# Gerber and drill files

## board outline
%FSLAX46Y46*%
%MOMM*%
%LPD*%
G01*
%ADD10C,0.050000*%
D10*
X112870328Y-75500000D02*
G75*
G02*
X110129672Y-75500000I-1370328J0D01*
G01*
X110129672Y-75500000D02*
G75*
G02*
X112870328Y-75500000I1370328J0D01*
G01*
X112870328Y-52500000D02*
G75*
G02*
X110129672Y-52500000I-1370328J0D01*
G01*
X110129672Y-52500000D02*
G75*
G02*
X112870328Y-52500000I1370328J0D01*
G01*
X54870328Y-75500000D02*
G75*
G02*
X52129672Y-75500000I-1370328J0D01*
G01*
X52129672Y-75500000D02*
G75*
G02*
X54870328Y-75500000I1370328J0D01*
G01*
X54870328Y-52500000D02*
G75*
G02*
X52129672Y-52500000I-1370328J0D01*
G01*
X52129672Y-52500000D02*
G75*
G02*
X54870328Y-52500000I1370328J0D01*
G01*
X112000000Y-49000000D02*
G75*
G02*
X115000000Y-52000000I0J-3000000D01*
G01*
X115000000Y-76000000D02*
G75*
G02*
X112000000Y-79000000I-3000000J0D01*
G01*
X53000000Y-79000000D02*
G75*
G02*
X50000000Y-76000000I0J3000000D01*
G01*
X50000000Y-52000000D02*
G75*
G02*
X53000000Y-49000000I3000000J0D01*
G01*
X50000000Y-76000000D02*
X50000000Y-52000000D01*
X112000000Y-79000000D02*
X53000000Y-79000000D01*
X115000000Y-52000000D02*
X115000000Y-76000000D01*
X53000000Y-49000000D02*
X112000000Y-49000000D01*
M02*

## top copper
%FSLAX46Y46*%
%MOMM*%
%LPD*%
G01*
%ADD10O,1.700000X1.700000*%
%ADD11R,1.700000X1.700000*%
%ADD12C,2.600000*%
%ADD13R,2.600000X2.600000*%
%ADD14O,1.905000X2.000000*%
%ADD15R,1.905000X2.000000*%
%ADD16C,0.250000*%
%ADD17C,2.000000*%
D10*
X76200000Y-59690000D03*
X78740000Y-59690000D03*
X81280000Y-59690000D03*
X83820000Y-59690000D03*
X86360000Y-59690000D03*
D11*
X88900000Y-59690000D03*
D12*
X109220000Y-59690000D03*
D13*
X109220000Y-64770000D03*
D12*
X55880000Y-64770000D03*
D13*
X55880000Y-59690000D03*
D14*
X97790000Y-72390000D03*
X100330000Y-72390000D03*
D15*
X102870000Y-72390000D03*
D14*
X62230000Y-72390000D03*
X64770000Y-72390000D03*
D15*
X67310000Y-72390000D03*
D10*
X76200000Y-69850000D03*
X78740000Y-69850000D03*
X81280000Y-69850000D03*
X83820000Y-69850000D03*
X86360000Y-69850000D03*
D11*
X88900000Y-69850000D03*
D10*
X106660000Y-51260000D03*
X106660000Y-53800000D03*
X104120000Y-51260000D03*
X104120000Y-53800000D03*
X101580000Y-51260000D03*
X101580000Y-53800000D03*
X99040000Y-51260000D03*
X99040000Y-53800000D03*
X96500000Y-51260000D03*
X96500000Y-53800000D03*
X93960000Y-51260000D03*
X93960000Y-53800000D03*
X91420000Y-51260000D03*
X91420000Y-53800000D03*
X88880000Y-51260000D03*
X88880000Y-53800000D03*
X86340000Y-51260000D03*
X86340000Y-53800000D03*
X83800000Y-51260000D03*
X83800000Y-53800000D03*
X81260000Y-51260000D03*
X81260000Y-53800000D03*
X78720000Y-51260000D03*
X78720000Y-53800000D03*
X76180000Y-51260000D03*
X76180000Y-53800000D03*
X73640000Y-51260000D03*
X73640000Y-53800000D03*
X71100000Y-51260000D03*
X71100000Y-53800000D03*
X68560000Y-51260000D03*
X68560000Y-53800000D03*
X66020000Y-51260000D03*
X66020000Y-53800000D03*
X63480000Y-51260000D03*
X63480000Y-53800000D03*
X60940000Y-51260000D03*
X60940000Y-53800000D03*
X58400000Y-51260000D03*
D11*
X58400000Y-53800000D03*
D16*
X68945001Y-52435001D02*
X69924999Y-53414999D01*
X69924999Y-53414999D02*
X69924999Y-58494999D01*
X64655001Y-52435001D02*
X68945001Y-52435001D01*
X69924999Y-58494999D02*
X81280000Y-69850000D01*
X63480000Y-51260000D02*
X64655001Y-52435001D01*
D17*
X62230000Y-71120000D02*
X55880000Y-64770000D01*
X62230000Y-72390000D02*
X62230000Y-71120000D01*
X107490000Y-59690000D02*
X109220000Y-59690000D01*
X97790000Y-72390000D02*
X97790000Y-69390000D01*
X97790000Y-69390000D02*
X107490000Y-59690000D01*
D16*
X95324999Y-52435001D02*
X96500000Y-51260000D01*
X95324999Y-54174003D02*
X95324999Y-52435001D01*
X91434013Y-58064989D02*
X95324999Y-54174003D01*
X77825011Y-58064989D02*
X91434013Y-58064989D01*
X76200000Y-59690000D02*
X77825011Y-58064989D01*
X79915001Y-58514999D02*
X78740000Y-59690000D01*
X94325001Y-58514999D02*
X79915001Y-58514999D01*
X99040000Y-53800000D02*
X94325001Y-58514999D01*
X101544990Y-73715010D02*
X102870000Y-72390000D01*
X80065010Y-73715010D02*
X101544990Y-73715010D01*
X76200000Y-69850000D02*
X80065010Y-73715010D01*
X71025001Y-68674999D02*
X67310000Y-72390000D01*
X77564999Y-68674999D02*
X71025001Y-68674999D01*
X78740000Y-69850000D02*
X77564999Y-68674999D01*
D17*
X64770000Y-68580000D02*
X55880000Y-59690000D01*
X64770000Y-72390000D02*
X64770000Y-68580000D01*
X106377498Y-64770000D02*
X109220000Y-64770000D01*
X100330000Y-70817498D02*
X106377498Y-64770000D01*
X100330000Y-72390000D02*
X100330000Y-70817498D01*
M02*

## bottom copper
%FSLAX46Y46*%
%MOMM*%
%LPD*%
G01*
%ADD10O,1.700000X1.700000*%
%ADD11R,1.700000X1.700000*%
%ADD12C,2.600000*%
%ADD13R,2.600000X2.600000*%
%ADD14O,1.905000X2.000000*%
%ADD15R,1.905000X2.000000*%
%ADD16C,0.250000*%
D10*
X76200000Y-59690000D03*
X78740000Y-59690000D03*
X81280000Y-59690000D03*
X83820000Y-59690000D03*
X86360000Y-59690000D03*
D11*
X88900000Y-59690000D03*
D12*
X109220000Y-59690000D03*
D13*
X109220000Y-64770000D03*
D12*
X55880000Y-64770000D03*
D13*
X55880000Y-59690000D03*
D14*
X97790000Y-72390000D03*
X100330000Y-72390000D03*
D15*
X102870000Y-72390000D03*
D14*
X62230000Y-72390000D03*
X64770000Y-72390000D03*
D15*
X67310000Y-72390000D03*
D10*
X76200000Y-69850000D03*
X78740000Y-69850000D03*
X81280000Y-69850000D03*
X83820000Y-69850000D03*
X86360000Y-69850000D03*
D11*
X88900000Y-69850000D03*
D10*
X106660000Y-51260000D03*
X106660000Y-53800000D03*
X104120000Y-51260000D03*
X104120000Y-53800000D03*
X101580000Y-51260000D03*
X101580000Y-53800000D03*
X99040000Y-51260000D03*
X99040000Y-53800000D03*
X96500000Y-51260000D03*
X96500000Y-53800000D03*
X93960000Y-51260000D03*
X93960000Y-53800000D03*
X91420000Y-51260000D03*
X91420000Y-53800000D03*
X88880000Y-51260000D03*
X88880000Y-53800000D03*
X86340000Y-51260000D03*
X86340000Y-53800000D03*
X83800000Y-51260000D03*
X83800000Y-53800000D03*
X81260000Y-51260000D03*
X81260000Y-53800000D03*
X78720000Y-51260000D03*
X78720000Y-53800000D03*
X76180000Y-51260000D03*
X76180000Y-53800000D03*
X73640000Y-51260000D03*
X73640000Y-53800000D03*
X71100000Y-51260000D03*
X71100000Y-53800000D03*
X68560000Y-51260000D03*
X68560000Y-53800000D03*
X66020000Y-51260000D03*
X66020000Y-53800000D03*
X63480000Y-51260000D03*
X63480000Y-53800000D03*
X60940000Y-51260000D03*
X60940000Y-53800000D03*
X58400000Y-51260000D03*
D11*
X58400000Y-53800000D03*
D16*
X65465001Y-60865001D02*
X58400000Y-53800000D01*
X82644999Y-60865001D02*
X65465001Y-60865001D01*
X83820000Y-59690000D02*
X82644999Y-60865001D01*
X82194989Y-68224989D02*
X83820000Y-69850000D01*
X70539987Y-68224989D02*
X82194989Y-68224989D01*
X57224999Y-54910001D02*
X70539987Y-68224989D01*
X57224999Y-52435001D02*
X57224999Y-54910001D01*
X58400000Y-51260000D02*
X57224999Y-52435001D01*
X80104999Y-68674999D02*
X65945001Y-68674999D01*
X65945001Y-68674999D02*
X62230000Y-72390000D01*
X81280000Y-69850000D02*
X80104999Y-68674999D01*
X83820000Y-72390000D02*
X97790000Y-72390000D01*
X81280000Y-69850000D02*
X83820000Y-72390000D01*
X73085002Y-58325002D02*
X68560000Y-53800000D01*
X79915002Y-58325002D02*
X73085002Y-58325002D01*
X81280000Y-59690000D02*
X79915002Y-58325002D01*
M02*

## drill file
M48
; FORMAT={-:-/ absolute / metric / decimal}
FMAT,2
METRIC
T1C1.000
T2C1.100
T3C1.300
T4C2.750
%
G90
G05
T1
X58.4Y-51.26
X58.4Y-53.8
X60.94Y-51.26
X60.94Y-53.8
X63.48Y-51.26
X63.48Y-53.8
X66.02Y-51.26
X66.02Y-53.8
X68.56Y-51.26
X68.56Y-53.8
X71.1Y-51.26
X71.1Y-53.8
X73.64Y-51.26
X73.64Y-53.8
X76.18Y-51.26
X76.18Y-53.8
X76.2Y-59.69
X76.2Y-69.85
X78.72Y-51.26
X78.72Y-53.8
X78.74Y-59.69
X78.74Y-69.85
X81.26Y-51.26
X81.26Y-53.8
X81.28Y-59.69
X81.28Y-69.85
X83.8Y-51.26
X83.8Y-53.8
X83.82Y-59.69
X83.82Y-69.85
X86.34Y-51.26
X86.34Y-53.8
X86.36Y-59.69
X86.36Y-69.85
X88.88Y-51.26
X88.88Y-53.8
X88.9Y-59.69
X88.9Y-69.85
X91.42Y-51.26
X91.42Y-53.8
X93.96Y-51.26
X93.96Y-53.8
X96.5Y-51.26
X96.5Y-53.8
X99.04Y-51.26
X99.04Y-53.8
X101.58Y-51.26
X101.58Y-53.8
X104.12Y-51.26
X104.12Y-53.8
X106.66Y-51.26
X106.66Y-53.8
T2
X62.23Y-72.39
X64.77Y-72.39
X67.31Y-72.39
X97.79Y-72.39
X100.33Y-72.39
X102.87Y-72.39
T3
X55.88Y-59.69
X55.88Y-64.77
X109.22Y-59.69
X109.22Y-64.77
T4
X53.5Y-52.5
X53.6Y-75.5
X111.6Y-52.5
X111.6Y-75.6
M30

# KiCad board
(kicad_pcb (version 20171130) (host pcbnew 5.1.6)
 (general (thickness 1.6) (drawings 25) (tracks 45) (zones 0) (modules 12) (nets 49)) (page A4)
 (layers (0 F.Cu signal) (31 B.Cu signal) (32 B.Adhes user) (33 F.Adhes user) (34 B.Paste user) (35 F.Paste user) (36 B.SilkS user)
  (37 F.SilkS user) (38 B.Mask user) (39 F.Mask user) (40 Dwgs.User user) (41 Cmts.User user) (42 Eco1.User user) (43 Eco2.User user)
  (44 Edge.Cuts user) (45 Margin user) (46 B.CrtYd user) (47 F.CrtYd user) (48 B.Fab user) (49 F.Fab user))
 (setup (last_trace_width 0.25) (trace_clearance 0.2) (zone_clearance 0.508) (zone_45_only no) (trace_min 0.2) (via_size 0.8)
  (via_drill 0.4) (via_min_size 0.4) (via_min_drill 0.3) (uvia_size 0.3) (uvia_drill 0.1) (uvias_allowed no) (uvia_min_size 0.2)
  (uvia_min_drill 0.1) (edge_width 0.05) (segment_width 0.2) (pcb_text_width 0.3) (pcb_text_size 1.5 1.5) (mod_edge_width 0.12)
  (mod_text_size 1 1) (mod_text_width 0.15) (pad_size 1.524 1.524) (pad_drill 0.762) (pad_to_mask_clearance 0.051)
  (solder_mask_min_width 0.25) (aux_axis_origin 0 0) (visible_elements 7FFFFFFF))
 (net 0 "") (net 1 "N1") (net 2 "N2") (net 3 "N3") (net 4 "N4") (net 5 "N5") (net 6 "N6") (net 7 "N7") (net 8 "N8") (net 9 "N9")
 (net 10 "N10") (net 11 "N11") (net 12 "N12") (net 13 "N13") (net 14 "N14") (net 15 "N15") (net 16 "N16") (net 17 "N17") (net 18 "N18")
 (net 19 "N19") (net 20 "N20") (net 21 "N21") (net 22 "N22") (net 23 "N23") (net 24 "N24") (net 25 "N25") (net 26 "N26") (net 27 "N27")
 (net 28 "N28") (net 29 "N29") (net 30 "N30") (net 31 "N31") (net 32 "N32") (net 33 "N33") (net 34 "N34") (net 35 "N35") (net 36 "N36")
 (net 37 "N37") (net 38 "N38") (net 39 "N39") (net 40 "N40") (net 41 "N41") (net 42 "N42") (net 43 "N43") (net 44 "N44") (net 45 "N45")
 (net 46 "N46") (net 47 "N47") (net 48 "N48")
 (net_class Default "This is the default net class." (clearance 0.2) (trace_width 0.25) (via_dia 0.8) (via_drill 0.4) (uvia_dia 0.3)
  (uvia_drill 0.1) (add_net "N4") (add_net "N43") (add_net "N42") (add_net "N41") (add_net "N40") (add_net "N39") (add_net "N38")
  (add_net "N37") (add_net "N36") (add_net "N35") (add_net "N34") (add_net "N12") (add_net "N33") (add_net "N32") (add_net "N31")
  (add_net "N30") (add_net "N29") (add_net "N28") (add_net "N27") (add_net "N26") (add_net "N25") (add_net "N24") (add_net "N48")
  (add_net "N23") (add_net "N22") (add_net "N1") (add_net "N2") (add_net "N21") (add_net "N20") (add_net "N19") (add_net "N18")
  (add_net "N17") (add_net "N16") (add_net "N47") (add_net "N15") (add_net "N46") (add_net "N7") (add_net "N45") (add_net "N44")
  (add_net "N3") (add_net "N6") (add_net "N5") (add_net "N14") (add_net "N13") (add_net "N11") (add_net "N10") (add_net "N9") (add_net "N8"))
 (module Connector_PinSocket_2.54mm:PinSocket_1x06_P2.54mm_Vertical (layer F.Cu) (at 88.9 59.69 270)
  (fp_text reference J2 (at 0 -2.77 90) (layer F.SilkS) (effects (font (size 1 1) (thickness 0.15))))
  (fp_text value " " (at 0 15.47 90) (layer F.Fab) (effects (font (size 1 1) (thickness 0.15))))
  (pad 6 thru_hole oval (at 0 12.7 270) (size 1.7 1.7) (drill 1) (layers *.Cu *.Mask) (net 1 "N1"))
  (pad 5 thru_hole oval (at 0 10.16 270) (size 1.7 1.7) (drill 1) (layers *.Cu *.Mask) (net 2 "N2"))
  (pad 4 thru_hole oval (at 0 7.62 270) (size 1.7 1.7) (drill 1) (layers *.Cu *.Mask) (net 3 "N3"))
  (pad 3 thru_hole oval (at 0 5.08 270) (size 1.7 1.7) (drill 1) (layers *.Cu *.Mask) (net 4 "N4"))
  (pad 2 thru_hole oval (at 0 2.54 270) (size 1.7 1.7) (drill 1) (layers *.Cu *.Mask) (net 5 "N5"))
  (pad 1 thru_hole rect (at 0 0 270) (size 1.7 1.7) (drill 1) (layers *.Cu *.Mask) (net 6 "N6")))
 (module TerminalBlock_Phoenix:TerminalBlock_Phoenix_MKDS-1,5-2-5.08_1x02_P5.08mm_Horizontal (layer F.Cu) (at 109.22 64.77 90)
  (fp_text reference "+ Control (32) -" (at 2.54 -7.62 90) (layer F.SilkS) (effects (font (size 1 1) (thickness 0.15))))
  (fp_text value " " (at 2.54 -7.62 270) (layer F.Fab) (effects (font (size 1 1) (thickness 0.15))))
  (pad 2 thru_hole circle (at 5.08 0 90) (size 2.6 2.6) (drill 1.3) (layers *.Cu *.Mask) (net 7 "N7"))
  (pad 1 thru_hole rect (at 0 0 90) (size 2.6 2.6) (drill 1.3) (layers *.Cu *.Mask) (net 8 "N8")))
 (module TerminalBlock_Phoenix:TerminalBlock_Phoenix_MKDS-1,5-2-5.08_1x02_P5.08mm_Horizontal (layer F.Cu) (at 55.88 59.69 270)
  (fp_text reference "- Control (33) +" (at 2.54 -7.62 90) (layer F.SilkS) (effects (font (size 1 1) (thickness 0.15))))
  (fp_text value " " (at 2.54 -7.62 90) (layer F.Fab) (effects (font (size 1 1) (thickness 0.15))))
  (pad 2 thru_hole circle (at 5.08 0 270) (size 2.6 2.6) (drill 1.3) (layers *.Cu *.Mask) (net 7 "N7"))
  (pad 1 thru_hole rect (at 0 0 270) (size 2.6 2.6) (drill 1.3) (layers *.Cu *.Mask) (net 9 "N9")))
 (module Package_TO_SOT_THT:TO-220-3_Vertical (layer F.Cu) (at 102.87 72.39 180)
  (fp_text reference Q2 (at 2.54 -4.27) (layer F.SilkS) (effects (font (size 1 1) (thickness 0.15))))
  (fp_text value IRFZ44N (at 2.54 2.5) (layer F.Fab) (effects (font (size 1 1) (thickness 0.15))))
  (pad 3 thru_hole oval (at 5.08 0 180) (size 1.905 2) (drill 1.1) (layers *.Cu *.Mask) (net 7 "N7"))
  (pad 2 thru_hole oval (at 2.54 0 180) (size 1.905 2) (drill 1.1) (layers *.Cu *.Mask) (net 8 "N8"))
  (pad 1 thru_hole rect (at 0 0 180) (size 1.905 2) (drill 1.1) (layers *.Cu *.Mask) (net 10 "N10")))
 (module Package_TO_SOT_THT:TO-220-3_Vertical (layer F.Cu) (at 67.31 72.39 180)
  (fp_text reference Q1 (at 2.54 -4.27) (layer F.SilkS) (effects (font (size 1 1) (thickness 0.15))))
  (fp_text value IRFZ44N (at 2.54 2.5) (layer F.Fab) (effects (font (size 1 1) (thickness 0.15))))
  (pad 3 thru_hole oval (at 5.08 0 180) (size 1.905 2) (drill 1.1) (layers *.Cu *.Mask) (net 7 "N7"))
  (pad 2 thru_hole oval (at 2.54 0 180) (size 1.905 2) (drill 1.1) (layers *.Cu *.Mask) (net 9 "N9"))
  (pad 1 thru_hole rect (at 0 0 180) (size 1.905 2) (drill 1.1) (layers *.Cu *.Mask) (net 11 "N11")))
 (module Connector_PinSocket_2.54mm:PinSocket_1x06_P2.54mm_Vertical (layer F.Cu) (at 88.9 69.85 270)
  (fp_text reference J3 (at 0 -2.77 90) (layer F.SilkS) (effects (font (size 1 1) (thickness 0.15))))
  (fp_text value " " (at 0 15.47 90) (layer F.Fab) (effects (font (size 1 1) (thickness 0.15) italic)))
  (pad 6 thru_hole oval (at 0 12.7 270) (size 1.7 1.7) (drill 1) (layers *.Cu *.Mask) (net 10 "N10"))
  (pad 5 thru_hole oval (at 0 10.16 270) (size 1.7 1.7) (drill 1) (layers *.Cu *.Mask) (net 11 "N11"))
  (pad 4 thru_hole oval (at 0 7.62 270) (size 1.7 1.7) (drill 1) (layers *.Cu *.Mask) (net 7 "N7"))
  (pad 3 thru_hole oval (at 0 5.08 270) (size 1.7 1.7) (drill 1) (layers *.Cu *.Mask) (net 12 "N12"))
  (pad 2 thru_hole oval (at 0 2.54 270) (size 1.7 1.7) (drill 1) (layers *.Cu *.Mask) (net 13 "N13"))
  (pad 1 thru_hole rect (at 0 0 270) (size 1.7 1.7) (drill 1) (layers *.Cu *.Mask) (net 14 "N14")))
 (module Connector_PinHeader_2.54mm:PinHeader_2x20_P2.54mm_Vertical (layer F.Cu) (at 58.4 53.8 90)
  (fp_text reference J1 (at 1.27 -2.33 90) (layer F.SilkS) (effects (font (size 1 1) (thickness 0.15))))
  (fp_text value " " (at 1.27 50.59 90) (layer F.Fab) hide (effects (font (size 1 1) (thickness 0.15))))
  (pad 40 thru_hole oval (at 2.54 48.26 90) (size 1.7 1.7) (drill 1) (layers *.Cu *.Mask) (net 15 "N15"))
  (pad 39 thru_hole oval (at 0 48.26 90) (size 1.7 1.7) (drill 1) (layers *.Cu *.Mask) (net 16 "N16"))
  (pad 38 thru_hole oval (at 2.54 45.72 90) (size 1.7 1.7) (drill 1) (layers *.Cu *.Mask) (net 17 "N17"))
  (pad 37 thru_hole oval (at 0 45.72 90) (size 1.7 1.7) (drill 1) (layers *.Cu *.Mask) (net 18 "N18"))
  (pad 36 thru_hole oval (at 2.54 43.18 90) (size 1.7 1.7) (drill 1) (layers *.Cu *.Mask) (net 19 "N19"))
  (pad 35 thru_hole oval (at 0 43.18 90) (size 1.7 1.7) (drill 1) (layers *.Cu *.Mask) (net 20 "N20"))
  (pad 34 thru_hole oval (at 2.54 40.64 90) (size 1.7 1.7) (drill 1) (layers *.Cu *.Mask) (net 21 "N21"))
  (pad 33 thru_hole oval (at 0 40.64 90) (size 1.7 1.7) (drill 1) (layers *.Cu *.Mask) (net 2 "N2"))
  (pad 32 thru_hole oval (at 2.54 38.1 90) (size 1.7 1.7) (drill 1) (layers *.Cu *.Mask) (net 1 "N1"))
  (pad 31 thru_hole oval (at 0 38.1 90) (size 1.7 1.7) (drill 1) (layers *.Cu *.Mask) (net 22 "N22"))
  (pad 30 thru_hole oval (at 2.54 35.56 90) (size 1.7 1.7) (drill 1) (layers *.Cu *.Mask) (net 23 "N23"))
  (pad 29 thru_hole oval (at 0 35.56 90) (size 1.7 1.7) (drill 1) (layers *.Cu *.Mask) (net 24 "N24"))
  (pad 28 thru_hole oval (at 2.54 33.02 90) (size 1.7 1.7) (drill 1) (layers *.Cu *.Mask) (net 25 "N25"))
  (pad 27 thru_hole oval (at 0 33.02 90) (size 1.7 1.7) (drill 1) (layers *.Cu *.Mask) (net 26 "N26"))
  (pad 26 thru_hole oval (at 2.54 30.48 90) (size 1.7 1.7) (drill 1) (layers *.Cu *.Mask) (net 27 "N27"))
  (pad 25 thru_hole oval (at 0 30.48 90) (size 1.7 1.7) (drill 1) (layers *.Cu *.Mask) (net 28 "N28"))
  (pad 24 thru_hole oval (at 2.54 27.94 90) (size 1.7 1.7) (drill 1) (layers *.Cu *.Mask) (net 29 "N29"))
  (pad 23 thru_hole oval (at 0 27.94 90) (size 1.7 1.7) (drill 1) (layers *.Cu *.Mask) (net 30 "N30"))
  (pad 22 thru_hole oval (at 2.54 25.4 90) (size 1.7 1.7) (drill 1) (layers *.Cu *.Mask) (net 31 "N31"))
  (pad 21 thru_hole oval (at 0 25.4 90) (size 1.7 1.7) (drill 1) (layers *.Cu *.Mask) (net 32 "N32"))
  (pad 20 thru_hole oval (at 2.54 22.86 90) (size 1.7 1.7) (drill 1) (layers *.Cu *.Mask) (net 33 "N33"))
  (pad 19 thru_hole oval (at 0 22.86 90) (size 1.7 1.7) (drill 1) (layers *.Cu *.Mask) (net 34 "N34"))
  (pad 18 thru_hole oval (at 2.54 20.32 90) (size 1.7 1.7) (drill 1) (layers *.Cu *.Mask) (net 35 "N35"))
  (pad 17 thru_hole oval (at 0 20.32 90) (size 1.7 1.7) (drill 1) (layers *.Cu *.Mask) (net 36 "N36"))
  (pad 16 thru_hole oval (at 2.54 17.78 90) (size 1.7 1.7) (drill 1) (layers *.Cu *.Mask) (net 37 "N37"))
  (pad 15 thru_hole oval (at 0 17.78 90) (size 1.7 1.7) (drill 1) (layers *.Cu *.Mask) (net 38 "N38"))
  (pad 14 thru_hole oval (at 2.54 15.24 90) (size 1.7 1.7) (drill 1) (layers *.Cu *.Mask) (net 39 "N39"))
  (pad 13 thru_hole oval (at 0 15.24 90) (size 1.7 1.7) (drill 1) (layers *.Cu *.Mask) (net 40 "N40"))
  (pad 12 thru_hole oval (at 2.54 12.7 90) (size 1.7 1.7) (drill 1) (layers *.Cu *.Mask) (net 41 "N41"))
  (pad 11 thru_hole oval (at 0 12.7 90) (size 1.7 1.7) (drill 1) (layers *.Cu *.Mask) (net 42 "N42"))
  (pad 10 thru_hole oval (at 2.54 10.16 90) (size 1.7 1.7) (drill 1) (layers *.Cu *.Mask) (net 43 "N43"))
  (pad 9 thru_hole oval (at 0 10.16 90) (size 1.7 1.7) (drill 1) (layers *.Cu *.Mask) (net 3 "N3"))
  (pad 8 thru_hole oval (at 2.54 7.62 90) (size 1.7 1.7) (drill 1) (layers *.Cu *.Mask) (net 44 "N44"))
  (pad 7 thru_hole oval (at 0 7.62 90) (size 1.7 1.7) (drill 1) (layers *.Cu *.Mask) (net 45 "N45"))
  (pad 6 thru_hole oval (at 2.54 5.08 90) (size 1.7 1.7) (drill 1) (layers *.Cu *.Mask) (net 7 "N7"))
  (pad 5 thru_hole oval (at 0 5.08 90) (size 1.7 1.7) (drill 1) (layers *.Cu *.Mask) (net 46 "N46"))
  (pad 4 thru_hole oval (at 2.54 2.54 90) (size 1.7 1.7) (drill 1) (layers *.Cu *.Mask) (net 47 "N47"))
  (pad 3 thru_hole oval (at 0 2.54 90) (size 1.7 1.7) (drill 1) (layers *.Cu *.Mask) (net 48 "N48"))
  (pad 2 thru_hole oval (at 2.54 0 90) (size 1.7 1.7) (drill 1) (layers *.Cu *.Mask) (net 12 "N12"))
  (pad 1 thru_hole rect (at 0 0 90) (size 1.7 1.7) (drill 1) (layers *.Cu *.Mask) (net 4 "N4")))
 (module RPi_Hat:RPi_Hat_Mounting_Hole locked (layer F.Cu) (at 53.5 52.5)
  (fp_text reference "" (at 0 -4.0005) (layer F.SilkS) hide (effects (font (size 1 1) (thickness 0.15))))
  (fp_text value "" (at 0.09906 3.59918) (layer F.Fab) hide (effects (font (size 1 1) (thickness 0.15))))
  (pad "" np_thru_hole circle (at 0 0) (size 2.75 2.75) (drill 2.75) (layers *.Cu *.Mask) (solder_mask_margin 1.725) (clearance 1.725)))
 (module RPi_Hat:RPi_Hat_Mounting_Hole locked (layer F.Cu) (at 53.6 75.5)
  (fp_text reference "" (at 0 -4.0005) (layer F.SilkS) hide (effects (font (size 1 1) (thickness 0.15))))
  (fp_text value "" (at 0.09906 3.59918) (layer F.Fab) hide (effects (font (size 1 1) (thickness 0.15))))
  (pad "" np_thru_hole circle (at 0 0) (size 2.75 2.75) (drill 2.75) (layers *.Cu *.Mask) (solder_mask_margin 1.725) (clearance 1.725)))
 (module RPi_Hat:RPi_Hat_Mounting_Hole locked (layer F.Cu) (at 111.6 75.6)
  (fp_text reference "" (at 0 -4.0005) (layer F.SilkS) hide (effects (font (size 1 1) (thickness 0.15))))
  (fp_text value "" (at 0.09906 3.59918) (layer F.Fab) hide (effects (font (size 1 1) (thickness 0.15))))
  (pad "" np_thru_hole circle (at 0 0) (size 2.75 2.75) (drill 2.75) (layers *.Cu *.Mask) (solder_mask_margin 1.725) (clearance 1.725)))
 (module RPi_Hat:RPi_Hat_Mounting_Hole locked (layer F.Cu) (at 111.6 52.5)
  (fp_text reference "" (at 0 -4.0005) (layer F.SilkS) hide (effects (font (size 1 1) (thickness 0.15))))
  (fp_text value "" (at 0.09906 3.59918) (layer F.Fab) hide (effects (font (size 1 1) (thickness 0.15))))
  (pad "" np_thru_hole circle (at 0 0) (size 2.75 2.75) (drill 2.75) (layers *.Cu *.Mask) (solder_mask_margin 1.725) (clearance 1.725)))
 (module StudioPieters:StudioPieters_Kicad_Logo (layer F.Cu) (at 202.8 170.6)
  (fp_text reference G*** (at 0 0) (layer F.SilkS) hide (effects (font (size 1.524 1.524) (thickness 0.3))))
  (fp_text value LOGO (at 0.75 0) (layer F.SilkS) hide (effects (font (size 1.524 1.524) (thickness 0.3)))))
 (gr_circle (center 111.5 75.5) (end 111.47 76.87) (layer Edge.Cuts) (width 0.05))
 (gr_circle (center 111.5 52.5) (end 111.47 53.87) (layer Edge.Cuts) (width 0.05))
 (gr_circle (center 53.5 75.5) (end 53.47 76.87) (layer Edge.Cuts) (width 0.05))
 (gr_circle (center 53.5 52.5) (end 53.47 53.87) (layer Edge.Cuts) (width 0.05))
 (gr_arc (start 112 52) (end 115 52) (angle -90) (layer Edge.Cuts) (width 0.05))
 (gr_arc (start 112 76) (end 112 79) (angle -90) (layer Edge.Cuts) (width 0.05))
 (gr_arc (start 53 76) (end 50 76) (angle -90) (layer Edge.Cuts) (width 0.05))
 (gr_arc (start 53 52) (end 53 49) (angle -90) (layer Edge.Cuts) (width 0.05))
 (gr_line (start 50 76) (end 50 52) (layer Edge.Cuts) (width 0.05))
 (gr_line (start 112 79) (end 53 79) (layer Edge.Cuts) (width 0.05))
 (gr_line (start 115 52) (end 115 76) (layer Edge.Cuts) (width 0.05))
 (gr_line (start 53 49) (end 112 49) (layer Edge.Cuts) (width 0.05))
 (segment (start 65.465001 60.865001) (end 58.4 53.8) (width 0.25) (layer B.Cu) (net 4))
 (segment (start 82.644999 60.865001) (end 65.465001 60.865001) (width 0.25) (layer B.Cu) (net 4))
 (segment (start 83.82 59.69) (end 82.644999 60.865001) (width 0.25) (layer B.Cu) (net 4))
 (segment (start 82.194989 68.224989) (end 83.82 69.85) (width 0.25) (layer B.Cu) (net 12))
 (segment (start 70.539987 68.224989) (end 82.194989 68.224989) (width 0.25) (layer B.Cu) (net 12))
 (segment (start 57.224999 54.910001) (end 70.539987 68.224989) (width 0.25) (layer B.Cu) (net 12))
 (segment (start 57.224999 52.435001) (end 57.224999 54.910001) (width 0.25) (layer B.Cu) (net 12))
 (segment (start 58.4 51.26) (end 57.224999 52.435001) (width 0.25) (layer B.Cu) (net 12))
 (segment (start 68.945001 52.435001) (end 69.924999 53.414999) (width 0.25) (layer F.Cu) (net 7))
 (segment (start 69.924999 53.414999) (end 69.924999 58.494999) (width 0.25) (layer F.Cu) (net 7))
 (segment (start 64.655001 52.435001) (end 68.945001 52.435001) (width 0.25) (layer F.Cu) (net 7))
 (segment (start 69.924999 58.494999) (end 81.28 69.85) (width 0.25) (layer F.Cu) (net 7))
 (segment (start 63.48 51.26) (end 64.655001 52.435001) (width 0.25) (layer F.Cu) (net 7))
 (segment (start 62.23 71.12) (end 55.88 64.77) (width 2) (layer F.Cu) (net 7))
 (segment (start 62.23 72.39) (end 62.23 71.12) (width 2) (layer F.Cu) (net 7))
 (segment (start 80.104999 68.674999) (end 65.945001 68.674999) (width 0.25) (layer B.Cu) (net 7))
 (segment (start 65.945001 68.674999) (end 62.23 72.39) (width 0.25) (layer B.Cu) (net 7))
 (segment (start 81.28 69.85) (end 80.104999 68.674999) (width 0.25) (layer B.Cu) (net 7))
 (segment (start 83.82 72.39) (end 97.79 72.39) (width 0.25) (layer B.Cu) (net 7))
 (segment (start 81.28 69.85) (end 83.82 72.39) (width 0.25) (layer B.Cu) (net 7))
 (segment (start 107.49 59.69) (end 109.22 59.69) (width 2) (layer F.Cu) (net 7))
 (segment (start 97.79 72.39) (end 97.79 69.39) (width 2) (layer F.Cu) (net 7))
 (segment (start 97.79 69.39) (end 107.49 59.69) (width 2) (layer F.Cu) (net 7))
 (segment (start 73.085002 58.325002) (end 68.56 53.8) (width 0.25) (layer B.Cu) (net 3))
 (segment (start 79.915002 58.325002) (end 73.085002 58.325002) (width 0.25) (layer B.Cu) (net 3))
 (segment (start 81.28 59.69) (end 79.915002 58.325002) (width 0.25) (layer B.Cu) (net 3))
 (segment (start 95.324999 52.435001) (end 96.5 51.26) (width 0.25) (layer F.Cu) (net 1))
 (segment (start 95.324999 54.174003) (end 95.324999 52.435001) (width 0.25) (layer F.Cu) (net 1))
 (segment (start 91.434013 58.064989) (end 95.324999 54.174003) (width 0.25) (layer F.Cu) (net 1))
 (segment (start 77.825011 58.064989) (end 91.434013 58.064989) (width 0.25) (layer F.Cu) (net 1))
 (segment (start 76.2 59.69) (end 77.825011 58.064989) (width 0.25) (layer F.Cu) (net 1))
 (segment (start 79.915001 58.514999) (end 78.74 59.69) (width 0.25) (layer F.Cu) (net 2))
 (segment (start 94.325001 58.514999) (end 79.915001 58.514999) (width 0.25) (layer F.Cu) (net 2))
 (segment (start 99.04 53.8) (end 94.325001 58.514999) (width 0.25) (layer F.Cu) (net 2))
 (segment (start 101.54499 73.71501) (end 102.87 72.39) (width 0.25) (layer F.Cu) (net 10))
 (segment (start 80.06501 73.71501) (end 101.54499 73.71501) (width 0.25) (layer F.Cu) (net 10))
 (segment (start 76.2 69.85) (end 80.06501 73.71501) (width 0.25) (layer F.Cu) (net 10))
 (segment (start 71.025001 68.674999) (end 67.31 72.39) (width 0.25) (layer F.Cu) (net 11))
 (segment (start 77.564999 68.674999) (end 71.025001 68.674999) (width 0.25) (layer F.Cu) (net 11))
 (segment (start 78.74 69.85) (end 77.564999 68.674999) (width 0.25) (layer F.Cu) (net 11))
 (segment (start 64.77 68.58) (end 55.88 59.69) (width 2) (layer F.Cu) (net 9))
 (segment (start 64.77 72.39) (end 64.77 68.58) (width 2) (layer F.Cu) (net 9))
 (segment (start 106.377498 64.77) (end 109.22 64.77) (width 2) (layer F.Cu) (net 8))
 (segment (start 100.33 70.817498) (end 106.377498 64.77) (width 2) (layer F.Cu) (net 8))
 (segment (start 100.33 72.39) (end 100.33 70.817498) (width 2) (layer F.Cu) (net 8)))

